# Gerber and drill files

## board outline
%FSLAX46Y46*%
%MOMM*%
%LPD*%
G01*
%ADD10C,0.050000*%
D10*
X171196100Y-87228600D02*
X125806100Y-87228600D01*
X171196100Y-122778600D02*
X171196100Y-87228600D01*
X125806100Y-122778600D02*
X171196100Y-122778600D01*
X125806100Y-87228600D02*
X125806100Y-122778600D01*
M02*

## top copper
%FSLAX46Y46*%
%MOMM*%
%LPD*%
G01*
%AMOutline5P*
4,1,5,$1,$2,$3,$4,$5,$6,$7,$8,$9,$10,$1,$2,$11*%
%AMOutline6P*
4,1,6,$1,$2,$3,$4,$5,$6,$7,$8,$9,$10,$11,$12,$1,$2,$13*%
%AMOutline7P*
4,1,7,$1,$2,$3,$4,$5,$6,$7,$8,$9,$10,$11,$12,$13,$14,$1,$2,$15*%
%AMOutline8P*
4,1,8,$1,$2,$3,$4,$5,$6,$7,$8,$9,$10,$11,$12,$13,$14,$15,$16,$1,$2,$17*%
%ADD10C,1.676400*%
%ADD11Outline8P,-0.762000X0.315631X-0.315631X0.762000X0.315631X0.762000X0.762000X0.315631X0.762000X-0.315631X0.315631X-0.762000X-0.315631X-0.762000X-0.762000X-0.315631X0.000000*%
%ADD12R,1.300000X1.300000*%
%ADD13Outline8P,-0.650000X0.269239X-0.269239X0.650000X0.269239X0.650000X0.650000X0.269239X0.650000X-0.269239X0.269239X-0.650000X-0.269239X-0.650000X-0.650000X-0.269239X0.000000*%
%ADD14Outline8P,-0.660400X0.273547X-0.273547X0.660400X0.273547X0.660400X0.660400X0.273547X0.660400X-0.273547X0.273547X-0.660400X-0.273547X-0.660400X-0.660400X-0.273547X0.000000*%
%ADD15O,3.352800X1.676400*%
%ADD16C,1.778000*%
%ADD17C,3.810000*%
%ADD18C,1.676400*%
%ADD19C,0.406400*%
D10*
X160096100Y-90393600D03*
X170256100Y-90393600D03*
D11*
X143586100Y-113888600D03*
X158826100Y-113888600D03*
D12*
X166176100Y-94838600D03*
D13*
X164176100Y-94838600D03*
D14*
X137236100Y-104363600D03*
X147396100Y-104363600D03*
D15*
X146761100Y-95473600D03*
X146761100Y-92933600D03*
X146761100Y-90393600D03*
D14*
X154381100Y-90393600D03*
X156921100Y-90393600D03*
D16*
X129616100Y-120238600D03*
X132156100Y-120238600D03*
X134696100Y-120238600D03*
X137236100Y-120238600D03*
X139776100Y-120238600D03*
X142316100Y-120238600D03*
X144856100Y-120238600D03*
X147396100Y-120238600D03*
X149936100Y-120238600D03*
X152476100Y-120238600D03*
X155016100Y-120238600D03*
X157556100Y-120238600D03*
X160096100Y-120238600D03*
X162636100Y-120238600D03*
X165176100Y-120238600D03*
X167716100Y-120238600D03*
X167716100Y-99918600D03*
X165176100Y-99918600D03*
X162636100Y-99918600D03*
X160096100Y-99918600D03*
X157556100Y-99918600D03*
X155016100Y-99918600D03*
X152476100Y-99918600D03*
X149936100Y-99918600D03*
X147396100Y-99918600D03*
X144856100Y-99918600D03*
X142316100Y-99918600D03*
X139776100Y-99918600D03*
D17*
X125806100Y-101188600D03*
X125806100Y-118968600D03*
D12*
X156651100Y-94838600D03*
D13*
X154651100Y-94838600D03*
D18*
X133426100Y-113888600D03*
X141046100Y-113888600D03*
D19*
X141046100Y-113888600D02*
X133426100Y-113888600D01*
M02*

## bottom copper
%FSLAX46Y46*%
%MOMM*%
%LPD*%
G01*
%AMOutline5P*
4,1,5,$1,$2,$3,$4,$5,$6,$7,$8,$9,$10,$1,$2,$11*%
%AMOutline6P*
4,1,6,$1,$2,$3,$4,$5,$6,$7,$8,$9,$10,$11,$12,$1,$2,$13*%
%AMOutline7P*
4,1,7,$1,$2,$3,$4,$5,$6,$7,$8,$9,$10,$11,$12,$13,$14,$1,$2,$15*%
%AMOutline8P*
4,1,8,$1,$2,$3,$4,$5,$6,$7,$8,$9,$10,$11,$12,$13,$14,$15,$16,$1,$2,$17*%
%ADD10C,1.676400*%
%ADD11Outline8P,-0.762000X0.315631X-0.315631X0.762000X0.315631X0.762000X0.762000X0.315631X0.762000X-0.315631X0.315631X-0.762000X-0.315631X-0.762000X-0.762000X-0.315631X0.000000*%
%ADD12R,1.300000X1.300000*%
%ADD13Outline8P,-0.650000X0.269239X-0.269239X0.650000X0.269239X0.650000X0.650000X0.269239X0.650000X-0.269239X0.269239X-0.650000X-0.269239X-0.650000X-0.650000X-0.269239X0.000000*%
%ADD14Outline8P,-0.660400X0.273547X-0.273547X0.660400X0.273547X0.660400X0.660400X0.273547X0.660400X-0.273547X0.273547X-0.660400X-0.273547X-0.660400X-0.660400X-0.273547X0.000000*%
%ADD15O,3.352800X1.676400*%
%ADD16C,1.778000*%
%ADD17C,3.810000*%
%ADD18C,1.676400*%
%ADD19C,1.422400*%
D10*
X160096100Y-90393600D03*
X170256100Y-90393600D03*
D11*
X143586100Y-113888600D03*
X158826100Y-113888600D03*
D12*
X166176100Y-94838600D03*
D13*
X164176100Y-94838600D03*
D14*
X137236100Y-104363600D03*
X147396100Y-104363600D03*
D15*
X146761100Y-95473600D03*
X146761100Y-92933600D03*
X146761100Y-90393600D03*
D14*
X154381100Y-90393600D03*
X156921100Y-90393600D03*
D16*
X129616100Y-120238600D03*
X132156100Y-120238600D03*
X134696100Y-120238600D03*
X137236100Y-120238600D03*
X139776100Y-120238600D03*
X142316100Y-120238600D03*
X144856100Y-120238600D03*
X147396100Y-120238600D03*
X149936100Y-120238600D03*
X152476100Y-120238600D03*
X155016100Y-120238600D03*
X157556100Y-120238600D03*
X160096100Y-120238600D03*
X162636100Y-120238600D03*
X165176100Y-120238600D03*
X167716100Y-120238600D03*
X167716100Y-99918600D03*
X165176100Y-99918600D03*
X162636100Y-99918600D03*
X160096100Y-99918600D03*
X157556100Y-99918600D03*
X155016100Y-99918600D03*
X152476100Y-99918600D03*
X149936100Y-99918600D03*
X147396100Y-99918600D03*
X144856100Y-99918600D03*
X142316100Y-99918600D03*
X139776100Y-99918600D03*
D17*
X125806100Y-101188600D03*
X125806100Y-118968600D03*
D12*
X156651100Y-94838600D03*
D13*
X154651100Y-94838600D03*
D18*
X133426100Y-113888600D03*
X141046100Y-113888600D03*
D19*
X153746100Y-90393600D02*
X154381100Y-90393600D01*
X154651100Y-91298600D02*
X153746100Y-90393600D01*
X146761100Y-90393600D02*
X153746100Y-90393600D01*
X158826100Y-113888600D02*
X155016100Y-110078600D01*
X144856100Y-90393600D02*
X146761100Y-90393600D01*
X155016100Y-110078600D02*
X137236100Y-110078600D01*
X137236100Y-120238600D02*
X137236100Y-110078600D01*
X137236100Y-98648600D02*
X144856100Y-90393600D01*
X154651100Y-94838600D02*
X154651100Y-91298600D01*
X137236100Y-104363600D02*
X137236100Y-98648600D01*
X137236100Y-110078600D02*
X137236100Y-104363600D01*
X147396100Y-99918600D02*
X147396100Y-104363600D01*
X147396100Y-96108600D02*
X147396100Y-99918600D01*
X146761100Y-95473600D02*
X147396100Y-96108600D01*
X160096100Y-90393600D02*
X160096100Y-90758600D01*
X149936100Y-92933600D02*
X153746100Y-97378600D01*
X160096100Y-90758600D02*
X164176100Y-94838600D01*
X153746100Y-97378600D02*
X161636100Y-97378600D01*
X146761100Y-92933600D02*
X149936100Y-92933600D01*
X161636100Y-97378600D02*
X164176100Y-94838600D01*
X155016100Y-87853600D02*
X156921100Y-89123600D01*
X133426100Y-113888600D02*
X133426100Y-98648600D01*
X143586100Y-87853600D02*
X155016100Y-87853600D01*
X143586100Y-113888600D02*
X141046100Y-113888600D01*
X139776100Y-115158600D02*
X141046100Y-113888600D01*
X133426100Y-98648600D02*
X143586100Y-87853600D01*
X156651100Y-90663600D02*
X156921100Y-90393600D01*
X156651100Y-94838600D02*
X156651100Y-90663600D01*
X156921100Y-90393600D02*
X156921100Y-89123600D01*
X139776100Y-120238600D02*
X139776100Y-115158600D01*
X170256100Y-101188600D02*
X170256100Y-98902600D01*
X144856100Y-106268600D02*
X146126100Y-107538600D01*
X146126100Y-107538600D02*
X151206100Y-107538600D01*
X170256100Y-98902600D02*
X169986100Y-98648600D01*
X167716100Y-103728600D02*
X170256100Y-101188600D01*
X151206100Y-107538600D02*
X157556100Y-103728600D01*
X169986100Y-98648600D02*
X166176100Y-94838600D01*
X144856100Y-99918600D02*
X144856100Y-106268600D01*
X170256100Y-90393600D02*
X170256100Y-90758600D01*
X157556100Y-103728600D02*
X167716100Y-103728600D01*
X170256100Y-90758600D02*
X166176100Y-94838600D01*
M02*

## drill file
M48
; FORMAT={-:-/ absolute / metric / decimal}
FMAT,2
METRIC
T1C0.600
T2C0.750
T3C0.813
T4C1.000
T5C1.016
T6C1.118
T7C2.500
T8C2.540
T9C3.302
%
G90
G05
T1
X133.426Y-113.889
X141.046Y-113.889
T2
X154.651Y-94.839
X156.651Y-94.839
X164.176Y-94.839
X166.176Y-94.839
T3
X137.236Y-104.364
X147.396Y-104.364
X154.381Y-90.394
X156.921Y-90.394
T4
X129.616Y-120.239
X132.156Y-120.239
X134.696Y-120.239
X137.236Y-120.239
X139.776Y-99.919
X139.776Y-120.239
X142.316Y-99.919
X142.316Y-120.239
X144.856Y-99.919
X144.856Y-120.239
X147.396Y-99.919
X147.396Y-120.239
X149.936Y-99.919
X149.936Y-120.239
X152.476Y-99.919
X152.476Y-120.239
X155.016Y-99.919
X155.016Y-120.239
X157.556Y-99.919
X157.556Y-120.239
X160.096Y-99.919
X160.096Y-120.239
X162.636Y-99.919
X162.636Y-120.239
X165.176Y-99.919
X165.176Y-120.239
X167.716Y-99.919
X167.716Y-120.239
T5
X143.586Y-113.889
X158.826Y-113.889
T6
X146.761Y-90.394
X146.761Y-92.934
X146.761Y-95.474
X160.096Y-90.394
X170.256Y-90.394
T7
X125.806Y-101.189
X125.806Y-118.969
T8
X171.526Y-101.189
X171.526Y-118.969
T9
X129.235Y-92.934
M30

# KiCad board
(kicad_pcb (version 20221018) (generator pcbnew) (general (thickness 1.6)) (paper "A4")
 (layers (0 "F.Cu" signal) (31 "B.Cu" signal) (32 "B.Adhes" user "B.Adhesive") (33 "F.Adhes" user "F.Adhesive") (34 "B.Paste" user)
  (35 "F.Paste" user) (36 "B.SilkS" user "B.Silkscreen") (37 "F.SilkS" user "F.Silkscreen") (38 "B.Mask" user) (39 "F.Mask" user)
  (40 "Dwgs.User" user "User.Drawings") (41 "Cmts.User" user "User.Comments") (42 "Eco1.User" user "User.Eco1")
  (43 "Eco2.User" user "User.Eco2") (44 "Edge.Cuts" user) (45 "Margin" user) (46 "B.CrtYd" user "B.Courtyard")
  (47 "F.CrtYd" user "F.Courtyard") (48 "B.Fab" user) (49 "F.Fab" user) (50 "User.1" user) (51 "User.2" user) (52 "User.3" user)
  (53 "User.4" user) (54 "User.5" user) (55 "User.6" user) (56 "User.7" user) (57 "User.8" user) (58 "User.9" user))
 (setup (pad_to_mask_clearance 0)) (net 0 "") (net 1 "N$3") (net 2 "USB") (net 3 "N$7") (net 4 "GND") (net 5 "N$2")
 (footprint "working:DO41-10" (layer "F.Cu") (at 165.1761 90.3936 180)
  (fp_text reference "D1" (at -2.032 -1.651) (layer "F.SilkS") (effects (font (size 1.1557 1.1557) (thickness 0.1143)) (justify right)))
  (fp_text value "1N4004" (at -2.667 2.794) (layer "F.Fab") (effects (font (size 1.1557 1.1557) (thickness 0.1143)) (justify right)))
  (pad "A" thru_hole circle (at 5.08 0 180) (size 1.6764 1.6764) (drill 1.1176) (layers "*.Cu" "*.Mask") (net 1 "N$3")
   (solder_mask_margin 0.1016))
  (pad "C" thru_hole circle (at -5.08 0 180) (size 1.6764 1.6764) (drill 1.1176) (layers "*.Cu" "*.Mask") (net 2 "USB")
   (solder_mask_margin 0.1016)))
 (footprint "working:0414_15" (layer "F.Cu") (at 151.2061 113.8886)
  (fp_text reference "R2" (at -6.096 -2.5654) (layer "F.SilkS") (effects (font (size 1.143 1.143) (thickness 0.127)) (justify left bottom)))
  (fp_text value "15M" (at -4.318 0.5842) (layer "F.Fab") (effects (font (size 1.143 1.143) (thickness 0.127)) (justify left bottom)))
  (pad "1" thru_hole roundrect (at -7.62 0) (size 1.524 1.524) (drill 1.016) (layers "*.Cu" "*.Mask") (roundrect_rratio 0.25)
   (chamfer_ratio 0.2928932188) (chamfer top_left top_right bottom_left bottom_right) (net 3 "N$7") (solder_mask_margin 0.1016)
   (thermal_bridge_angle 45))
  (pad "2" thru_hole roundrect (at 7.62 0) (size 1.524 1.524) (drill 1.016) (layers "*.Cu" "*.Mask") (roundrect_rratio 0.25)
   (chamfer_ratio 0.2928932188) (chamfer top_left top_right bottom_left bottom_right) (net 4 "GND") (solder_mask_margin 0.1016)
   (thermal_bridge_angle 45)))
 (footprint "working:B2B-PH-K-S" (layer "F.Cu") (at 165.1761 94.8386)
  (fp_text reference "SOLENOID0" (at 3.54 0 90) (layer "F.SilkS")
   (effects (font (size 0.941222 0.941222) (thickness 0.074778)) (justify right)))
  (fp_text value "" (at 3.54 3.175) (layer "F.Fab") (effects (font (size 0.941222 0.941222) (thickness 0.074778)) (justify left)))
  (pad "1" thru_hole rect (at 1 0) (size 1.3 1.3) (drill 0.75) (layers "*.Cu" "*.Mask") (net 2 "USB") (solder_mask_margin 0.1016)
   (thermal_bridge_angle 45))
  (pad "2" thru_hole roundrect (at -1 0) (size 1.3 1.3) (drill 0.75) (layers "*.Cu" "*.Mask") (roundrect_rratio 0.25)
   (chamfer_ratio 0.2928932188) (chamfer top_left top_right bottom_left bottom_right) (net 1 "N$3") (solder_mask_margin 0.1016)
   (thermal_bridge_angle 45)))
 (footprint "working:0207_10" (layer "F.Cu") (at 142.3161 104.3636)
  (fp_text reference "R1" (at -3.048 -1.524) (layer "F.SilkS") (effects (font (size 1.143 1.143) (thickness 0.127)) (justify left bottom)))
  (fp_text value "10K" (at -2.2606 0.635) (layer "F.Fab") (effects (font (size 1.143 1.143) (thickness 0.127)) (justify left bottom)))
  (pad "1" thru_hole roundrect (at -5.08 0) (size 1.3208 1.3208) (drill 0.8128) (layers "*.Cu" "*.Mask") (roundrect_rratio 0.25)
   (chamfer_ratio 0.2928932188) (chamfer top_left top_right bottom_left bottom_right) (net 4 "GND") (solder_mask_margin 0.1016)
   (thermal_bridge_angle 45))
  (pad "2" thru_hole roundrect (at 5.08 0) (size 1.3208 1.3208) (drill 0.8128) (layers "*.Cu" "*.Mask") (roundrect_rratio 0.25)
   (chamfer_ratio 0.2928932188) (chamfer top_left top_right bottom_left bottom_right) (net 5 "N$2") (solder_mask_margin 0.1016)
   (thermal_bridge_angle 45)))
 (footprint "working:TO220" (layer "F.Cu") (at 140.4111 92.9336 90)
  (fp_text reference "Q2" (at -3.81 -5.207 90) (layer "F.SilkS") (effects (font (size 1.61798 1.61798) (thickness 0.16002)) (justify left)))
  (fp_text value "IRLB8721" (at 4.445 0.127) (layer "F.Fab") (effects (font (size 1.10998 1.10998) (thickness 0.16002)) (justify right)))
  (pad "" np_thru_hole circle (at 0 -11.176 90) (size 3.302 3.302) (drill 3.302) (layers "*.Cu" "*.Mask"))
  (pad "1" thru_hole oval (at -2.54 6.35 180) (size 3.3528 1.6764) (drill 1.1176) (layers "*.Cu" "*.Mask") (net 5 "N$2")
   (solder_mask_margin 0.1016) (thermal_bridge_angle 45))
  (pad "2" thru_hole oval (at 0 6.35 180) (size 3.3528 1.6764) (drill 1.1176) (layers "*.Cu" "*.Mask") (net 1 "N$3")
   (solder_mask_margin 0.1016) (thermal_bridge_angle 45))
  (pad "3" thru_hole oval (at 2.54 6.35 180) (size 3.3528 1.6764) (drill 1.1176) (layers "*.Cu" "*.Mask") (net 4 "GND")
   (solder_mask_margin 0.1016) (thermal_bridge_angle 45))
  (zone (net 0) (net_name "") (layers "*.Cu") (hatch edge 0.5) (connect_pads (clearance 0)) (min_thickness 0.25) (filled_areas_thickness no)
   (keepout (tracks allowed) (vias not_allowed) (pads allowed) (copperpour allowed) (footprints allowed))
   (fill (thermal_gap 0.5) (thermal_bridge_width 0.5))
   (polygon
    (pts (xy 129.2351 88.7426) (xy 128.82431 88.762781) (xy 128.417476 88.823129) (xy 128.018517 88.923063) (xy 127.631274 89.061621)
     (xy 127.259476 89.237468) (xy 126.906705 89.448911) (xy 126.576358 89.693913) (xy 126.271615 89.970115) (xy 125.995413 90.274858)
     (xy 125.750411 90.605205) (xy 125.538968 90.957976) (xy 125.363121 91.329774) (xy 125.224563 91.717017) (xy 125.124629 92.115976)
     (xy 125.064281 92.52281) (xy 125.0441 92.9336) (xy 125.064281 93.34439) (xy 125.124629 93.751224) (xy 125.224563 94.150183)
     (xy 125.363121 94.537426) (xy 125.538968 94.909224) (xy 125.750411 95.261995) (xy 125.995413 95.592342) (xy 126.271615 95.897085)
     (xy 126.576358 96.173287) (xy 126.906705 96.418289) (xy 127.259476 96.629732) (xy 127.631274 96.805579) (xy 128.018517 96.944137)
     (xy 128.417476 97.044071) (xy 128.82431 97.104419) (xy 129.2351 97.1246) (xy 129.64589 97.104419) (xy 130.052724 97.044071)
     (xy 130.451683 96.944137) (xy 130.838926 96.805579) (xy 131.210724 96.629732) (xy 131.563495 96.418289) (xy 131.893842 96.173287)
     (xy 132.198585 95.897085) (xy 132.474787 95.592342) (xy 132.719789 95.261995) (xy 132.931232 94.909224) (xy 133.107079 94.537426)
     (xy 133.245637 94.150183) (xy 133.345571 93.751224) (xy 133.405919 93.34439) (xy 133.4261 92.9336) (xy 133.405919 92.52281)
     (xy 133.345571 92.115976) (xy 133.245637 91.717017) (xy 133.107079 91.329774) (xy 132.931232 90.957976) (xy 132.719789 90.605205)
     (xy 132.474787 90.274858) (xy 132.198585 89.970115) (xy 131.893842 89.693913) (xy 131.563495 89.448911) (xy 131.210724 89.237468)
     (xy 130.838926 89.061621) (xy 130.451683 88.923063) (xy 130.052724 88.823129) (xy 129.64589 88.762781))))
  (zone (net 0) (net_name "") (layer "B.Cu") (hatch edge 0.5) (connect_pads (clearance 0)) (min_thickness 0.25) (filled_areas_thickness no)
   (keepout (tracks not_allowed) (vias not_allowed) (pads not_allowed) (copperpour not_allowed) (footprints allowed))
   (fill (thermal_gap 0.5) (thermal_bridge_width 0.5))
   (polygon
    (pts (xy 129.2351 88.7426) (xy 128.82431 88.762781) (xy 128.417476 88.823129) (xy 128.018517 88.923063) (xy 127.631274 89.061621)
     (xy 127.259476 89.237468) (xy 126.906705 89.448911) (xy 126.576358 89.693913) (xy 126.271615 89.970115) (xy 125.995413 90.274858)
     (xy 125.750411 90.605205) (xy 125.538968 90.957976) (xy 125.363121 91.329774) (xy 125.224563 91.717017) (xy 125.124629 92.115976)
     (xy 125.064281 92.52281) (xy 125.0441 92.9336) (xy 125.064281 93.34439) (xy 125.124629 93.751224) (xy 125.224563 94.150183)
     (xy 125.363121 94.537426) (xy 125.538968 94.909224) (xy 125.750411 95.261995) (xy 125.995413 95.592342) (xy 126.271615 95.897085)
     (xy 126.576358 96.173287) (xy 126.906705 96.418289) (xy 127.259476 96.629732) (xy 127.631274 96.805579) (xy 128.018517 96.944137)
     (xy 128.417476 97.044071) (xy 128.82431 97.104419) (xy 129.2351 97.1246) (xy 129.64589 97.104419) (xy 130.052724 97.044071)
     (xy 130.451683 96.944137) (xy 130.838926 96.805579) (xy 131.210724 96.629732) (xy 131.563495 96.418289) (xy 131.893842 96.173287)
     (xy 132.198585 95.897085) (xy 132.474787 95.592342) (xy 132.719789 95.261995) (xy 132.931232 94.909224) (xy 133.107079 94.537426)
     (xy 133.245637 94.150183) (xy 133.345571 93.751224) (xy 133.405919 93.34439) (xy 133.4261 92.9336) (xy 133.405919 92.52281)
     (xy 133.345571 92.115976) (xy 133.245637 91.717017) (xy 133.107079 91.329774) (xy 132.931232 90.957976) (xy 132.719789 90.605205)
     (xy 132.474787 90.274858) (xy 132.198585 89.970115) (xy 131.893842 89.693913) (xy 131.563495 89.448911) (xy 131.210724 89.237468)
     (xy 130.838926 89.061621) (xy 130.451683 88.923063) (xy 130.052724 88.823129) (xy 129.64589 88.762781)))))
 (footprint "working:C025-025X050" (layer "F.Cu") (at 155.6511 90.3936)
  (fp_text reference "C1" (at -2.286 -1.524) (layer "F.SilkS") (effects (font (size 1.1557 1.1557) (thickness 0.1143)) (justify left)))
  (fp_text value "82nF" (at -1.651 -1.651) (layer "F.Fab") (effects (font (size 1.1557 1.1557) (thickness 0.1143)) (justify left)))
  (pad "1" thru_hole roundrect (at -1.27 0) (size 1.3208 1.3208) (drill 0.8128) (layers "*.Cu" "*.Mask") (roundrect_rratio 0.25)
   (chamfer_ratio 0.2928932188) (chamfer top_left top_right bottom_left bottom_right) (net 4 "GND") (solder_mask_margin 0.1016)
   (thermal_bridge_angle 45))
  (pad "2" thru_hole roundrect (at 1.27 0) (size 1.3208 1.3208) (drill 0.8128) (layers "*.Cu" "*.Mask") (roundrect_rratio 0.25)
   (chamfer_ratio 0.2928932188) (chamfer top_left top_right bottom_left bottom_right) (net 3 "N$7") (solder_mask_margin 0.1016)
   (thermal_bridge_angle 45)))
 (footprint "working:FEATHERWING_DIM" (layer "F.Cu") (at 123.2661 121.5086)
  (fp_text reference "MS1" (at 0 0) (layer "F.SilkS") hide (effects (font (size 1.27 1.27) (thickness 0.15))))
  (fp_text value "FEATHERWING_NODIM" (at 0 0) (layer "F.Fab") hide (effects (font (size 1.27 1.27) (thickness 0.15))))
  (pad "" np_thru_hole circle (at 48.26 -20.32) (size 2.54 2.54) (drill 2.54) (layers "*.Cu" "*.Mask"))
  (pad "" np_thru_hole circle (at 48.26 -2.54) (size 2.54 2.54) (drill 2.54) (layers "*.Cu" "*.Mask"))
  (pad "1" thru_hole circle (at 6.35 -1.27) (size 1.778 1.778) (drill 1) (layers "*.Cu" "*.Mask") (solder_mask_margin 0.1016))
  (pad "2" thru_hole circle (at 8.89 -1.27) (size 1.778 1.778) (drill 1) (layers "*.Cu" "*.Mask") (solder_mask_margin 0.1016))
  (pad "3" thru_hole circle (at 11.43 -1.27) (size 1.778 1.778) (drill 1) (layers "*.Cu" "*.Mask") (solder_mask_margin 0.1016))
  (pad "4" thru_hole circle (at 13.97 -1.27) (size 1.778 1.778) (drill 1) (layers "*.Cu" "*.Mask") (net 4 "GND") (solder_mask_margin 0.1016))
  (pad "5" thru_hole circle (at 16.51 -1.27) (size 1.778 1.778) (drill 1) (layers "*.Cu" "*.Mask") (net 3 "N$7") (solder_mask_margin 0.1016))
  (pad "6" thru_hole circle (at 19.05 -1.27) (size 1.778 1.778) (drill 1) (layers "*.Cu" "*.Mask") (solder_mask_margin 0.1016))
  (pad "7" thru_hole circle (at 21.59 -1.27) (size 1.778 1.778) (drill 1) (layers "*.Cu" "*.Mask") (solder_mask_margin 0.1016))
  (pad "8" thru_hole circle (at 24.13 -1.27) (size 1.778 1.778) (drill 1) (layers "*.Cu" "*.Mask") (solder_mask_margin 0.1016))
  (pad "9" thru_hole circle (at 26.67 -1.27) (size 1.778 1.778) (drill 1) (layers "*.Cu" "*.Mask") (solder_mask_margin 0.1016))
  (pad "10" thru_hole circle (at 29.21 -1.27) (size 1.778 1.778) (drill 1) (layers "*.Cu" "*.Mask") (solder_mask_margin 0.1016))
  (pad "11" thru_hole circle (at 31.75 -1.27) (size 1.778 1.778) (drill 1) (layers "*.Cu" "*.Mask") (solder_mask_margin 0.1016))
  (pad "12" thru_hole circle (at 34.29 -1.27) (size 1.778 1.778) (drill 1) (layers "*.Cu" "*.Mask") (solder_mask_margin 0.1016))
  (pad "13" thru_hole circle (at 36.83 -1.27) (size 1.778 1.778) (drill 1) (layers "*.Cu" "*.Mask") (solder_mask_margin 0.1016))
  (pad "14" thru_hole circle (at 39.37 -1.27) (size 1.778 1.778) (drill 1) (layers "*.Cu" "*.Mask") (solder_mask_margin 0.1016))
  (pad "15" thru_hole circle (at 41.91 -1.27) (size 1.778 1.778) (drill 1) (layers "*.Cu" "*.Mask") (solder_mask_margin 0.1016))
  (pad "16" thru_hole circle (at 44.45 -1.27) (size 1.778 1.778) (drill 1) (layers "*.Cu" "*.Mask") (solder_mask_margin 0.1016))
  (pad "17" thru_hole circle (at 44.45 -21.59) (size 1.778 1.778) (drill 1) (layers "*.Cu" "*.Mask") (solder_mask_margin 0.1016))
  (pad "18" thru_hole circle (at 41.91 -21.59) (size 1.778 1.778) (drill 1) (layers "*.Cu" "*.Mask") (solder_mask_margin 0.1016))
  (pad "19" thru_hole circle (at 39.37 -21.59) (size 1.778 1.778) (drill 1) (layers "*.Cu" "*.Mask") (solder_mask_margin 0.1016))
  (pad "20" thru_hole circle (at 36.83 -21.59) (size 1.778 1.778) (drill 1) (layers "*.Cu" "*.Mask") (solder_mask_margin 0.1016))
  (pad "21" thru_hole circle (at 34.29 -21.59) (size 1.778 1.778) (drill 1) (layers "*.Cu" "*.Mask") (solder_mask_margin 0.1016))
  (pad "22" thru_hole circle (at 31.75 -21.59) (size 1.778 1.778) (drill 1) (layers "*.Cu" "*.Mask") (solder_mask_margin 0.1016))
  (pad "23" thru_hole circle (at 29.21 -21.59) (size 1.778 1.778) (drill 1) (layers "*.Cu" "*.Mask") (solder_mask_margin 0.1016))
  (pad "24" thru_hole circle (at 26.67 -21.59) (size 1.778 1.778) (drill 1) (layers "*.Cu" "*.Mask") (solder_mask_margin 0.1016))
  (pad "25" thru_hole circle (at 24.13 -21.59) (size 1.778 1.778) (drill 1) (layers "*.Cu" "*.Mask") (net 5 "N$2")
   (solder_mask_margin 0.1016))
  (pad "26" thru_hole circle (at 21.59 -21.59) (size 1.778 1.778) (drill 1) (layers "*.Cu" "*.Mask") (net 2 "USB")
   (solder_mask_margin 0.1016))
  (pad "27" thru_hole circle (at 19.05 -21.59) (size 1.778 1.778) (drill 1) (layers "*.Cu" "*.Mask") (solder_mask_margin 0.1016))
  (pad "28" thru_hole circle (at 16.51 -21.59) (size 1.778 1.778) (drill 1) (layers "*.Cu" "*.Mask") (solder_mask_margin 0.1016))
  (pad "P$1" thru_hole circle (at 2.54 -20.32) (size 3.81 3.81) (drill 2.5) (layers "*.Cu" "*.Mask") (solder_mask_margin 0.1016))
  (pad "P$2" thru_hole circle (at 2.54 -2.54) (size 3.81 3.81) (drill 2.5) (layers "*.Cu" "*.Mask") (solder_mask_margin 0.1016)))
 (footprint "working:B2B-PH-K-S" (layer "F.Cu") (at 155.6511 94.8386)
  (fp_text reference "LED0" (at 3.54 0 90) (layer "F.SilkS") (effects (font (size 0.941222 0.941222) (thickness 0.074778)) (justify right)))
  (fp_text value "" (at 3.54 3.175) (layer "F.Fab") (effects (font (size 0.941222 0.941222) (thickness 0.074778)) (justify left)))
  (pad "1" thru_hole rect (at 1 0) (size 1.3 1.3) (drill 0.75) (layers "*.Cu" "*.Mask") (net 3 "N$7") (solder_mask_margin 0.1016)
   (thermal_bridge_angle 45))
  (pad "2" thru_hole roundrect (at -1 0) (size 1.3 1.3) (drill 0.75) (layers "*.Cu" "*.Mask") (roundrect_rratio 0.25)
   (chamfer_ratio 0.2928932188) (chamfer top_left top_right bottom_left bottom_right) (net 4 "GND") (solder_mask_margin 0.1016)
   (thermal_bridge_angle 45)))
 (gr_line (start 171.1961 87.2286) (end 125.8061 87.2286) (stroke (width 0.05) (type solid)) (layer "Edge.Cuts"))
 (gr_line (start 171.1961 122.7786) (end 171.1961 87.2286) (stroke (width 0.05) (type solid)) (layer "Edge.Cuts"))
 (gr_line (start 125.8061 122.7786) (end 171.1961 122.7786) (stroke (width 0.05) (type solid)) (layer "Edge.Cuts"))
 (gr_line (start 125.8061 87.2286) (end 125.8061 122.7786) (stroke (width 0.05) (type solid)) (layer "Edge.Cuts"))
 (segment (start 153.7461 90.3936) (end 154.3811 90.3936) (width 1.4224) (layer "B.Cu") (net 4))
 (segment (start 154.6511 91.2986) (end 153.7461 90.3936) (width 1.4224) (layer "B.Cu") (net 4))
 (segment (start 146.7611 90.3936) (end 153.7461 90.3936) (width 1.4224) (layer "B.Cu") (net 4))
 (segment (start 158.8261 113.8886) (end 155.0161 110.0786) (width 1.4224) (layer "B.Cu") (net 4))
 (segment (start 144.8561 90.3936) (end 146.7611 90.3936) (width 1.4224) (layer "B.Cu") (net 4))
 (segment (start 155.0161 110.0786) (end 137.2361 110.0786) (width 1.4224) (layer "B.Cu") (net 4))
 (segment (start 137.2361 120.2386) (end 137.2361 110.0786) (width 1.4224) (layer "B.Cu") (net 4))
 (segment (start 137.2361 98.6486) (end 144.8561 90.3936) (width 1.4224) (layer "B.Cu") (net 4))
 (segment (start 154.6511 94.8386) (end 154.6511 91.2986) (width 1.4224) (layer "B.Cu") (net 4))
 (segment (start 137.2361 104.3636) (end 137.2361 98.6486) (width 1.4224) (layer "B.Cu") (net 4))
 (segment (start 137.2361 110.0786) (end 137.2361 104.3636) (width 1.4224) (layer "B.Cu") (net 4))
 (segment (start 147.3961 99.9186) (end 147.3961 104.3636) (width 1.4224) (layer "B.Cu") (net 5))
 (segment (start 147.3961 96.1086) (end 147.3961 99.9186) (width 1.4224) (layer "B.Cu") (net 5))
 (segment (start 146.7611 95.4736) (end 147.3961 96.1086) (width 1.4224) (layer "B.Cu") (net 5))
 (segment (start 160.0961 90.3936) (end 160.0961 90.7586) (width 1.4224) (layer "B.Cu") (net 1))
 (segment (start 149.9361 92.9336) (end 153.7461 97.3786) (width 1.4224) (layer "B.Cu") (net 1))
 (segment (start 160.0961 90.7586) (end 164.1761 94.8386) (width 1.4224) (layer "B.Cu") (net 1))
 (segment (start 153.7461 97.3786) (end 161.6361 97.3786) (width 1.4224) (layer "B.Cu") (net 1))
 (segment (start 146.7611 92.9336) (end 149.9361 92.9336) (width 1.4224) (layer "B.Cu") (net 1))
 (segment (start 161.6361 97.3786) (end 164.1761 94.8386) (width 1.4224) (layer "B.Cu") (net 1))
 (segment (start 141.0461 113.8886) (end 133.4261 113.8886) (width 0.4064) (layer "F.Cu") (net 3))
 (via (at 133.4261 113.8886) (size 1.6764) (drill 0.6) (layers "F.Cu" "B.Cu") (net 3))
 (via (at 141.0461 113.8886) (size 1.6764) (drill 0.6) (layers "F.Cu" "B.Cu") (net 3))
 (segment (start 155.0161 87.8536) (end 156.9211 89.1236) (width 1.4224) (layer "B.Cu") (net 3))
 (segment (start 133.4261 113.8886) (end 133.4261 98.6486) (width 1.4224) (layer "B.Cu") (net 3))
 (segment (start 143.5861 87.8536) (end 155.0161 87.8536) (width 1.4224) (layer "B.Cu") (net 3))
 (segment (start 143.5861 113.8886) (end 141.0461 113.8886) (width 1.4224) (layer "B.Cu") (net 3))
 (segment (start 139.7761 115.1586) (end 141.0461 113.8886) (width 1.4224) (layer "B.Cu") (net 3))
 (segment (start 133.4261 98.6486) (end 143.5861 87.8536) (width 1.4224) (layer "B.Cu") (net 3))
 (segment (start 156.6511 90.6636) (end 156.9211 90.3936) (width 1.4224) (layer "B.Cu") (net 3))
 (segment (start 156.6511 94.8386) (end 156.6511 90.6636) (width 1.4224) (layer "B.Cu") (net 3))
 (segment (start 156.9211 90.3936) (end 156.9211 89.1236) (width 1.4224) (layer "B.Cu") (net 3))
 (segment (start 139.7761 120.2386) (end 139.7761 115.1586) (width 1.4224) (layer "B.Cu") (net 3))
 (segment (start 170.2561 101.1886) (end 170.2561 98.9026) (width 1.4224) (layer "B.Cu") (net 2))
 (segment (start 144.8561 106.2686) (end 146.1261 107.5386) (width 1.4224) (layer "B.Cu") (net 2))
 (segment (start 146.1261 107.5386) (end 151.2061 107.5386) (width 1.4224) (layer "B.Cu") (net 2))
 (segment (start 170.2561 98.9026) (end 169.9861 98.6486) (width 1.4224) (layer "B.Cu") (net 2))
 (segment (start 167.7161 103.7286) (end 170.2561 101.1886) (width 1.4224) (layer "B.Cu") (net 2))
 (segment (start 151.2061 107.5386) (end 157.5561 103.7286) (width 1.4224) (layer "B.Cu") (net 2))
 (segment (start 169.9861 98.6486) (end 166.1761 94.8386) (width 1.4224) (layer "B.Cu") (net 2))
 (segment (start 144.8561 99.9186) (end 144.8561 106.2686) (width 1.4224) (layer "B.Cu") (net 2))
 (segment (start 170.2561 90.3936) (end 170.2561 90.7586) (width 1.4224) (layer "B.Cu") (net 2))
 (segment (start 157.5561 103.7286) (end 167.7161 103.7286) (width 1.4224) (layer "B.Cu") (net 2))
 (segment (start 170.2561 90.7586) (end 166.1761 94.8386) (width 1.4224) (layer "B.Cu") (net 2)))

